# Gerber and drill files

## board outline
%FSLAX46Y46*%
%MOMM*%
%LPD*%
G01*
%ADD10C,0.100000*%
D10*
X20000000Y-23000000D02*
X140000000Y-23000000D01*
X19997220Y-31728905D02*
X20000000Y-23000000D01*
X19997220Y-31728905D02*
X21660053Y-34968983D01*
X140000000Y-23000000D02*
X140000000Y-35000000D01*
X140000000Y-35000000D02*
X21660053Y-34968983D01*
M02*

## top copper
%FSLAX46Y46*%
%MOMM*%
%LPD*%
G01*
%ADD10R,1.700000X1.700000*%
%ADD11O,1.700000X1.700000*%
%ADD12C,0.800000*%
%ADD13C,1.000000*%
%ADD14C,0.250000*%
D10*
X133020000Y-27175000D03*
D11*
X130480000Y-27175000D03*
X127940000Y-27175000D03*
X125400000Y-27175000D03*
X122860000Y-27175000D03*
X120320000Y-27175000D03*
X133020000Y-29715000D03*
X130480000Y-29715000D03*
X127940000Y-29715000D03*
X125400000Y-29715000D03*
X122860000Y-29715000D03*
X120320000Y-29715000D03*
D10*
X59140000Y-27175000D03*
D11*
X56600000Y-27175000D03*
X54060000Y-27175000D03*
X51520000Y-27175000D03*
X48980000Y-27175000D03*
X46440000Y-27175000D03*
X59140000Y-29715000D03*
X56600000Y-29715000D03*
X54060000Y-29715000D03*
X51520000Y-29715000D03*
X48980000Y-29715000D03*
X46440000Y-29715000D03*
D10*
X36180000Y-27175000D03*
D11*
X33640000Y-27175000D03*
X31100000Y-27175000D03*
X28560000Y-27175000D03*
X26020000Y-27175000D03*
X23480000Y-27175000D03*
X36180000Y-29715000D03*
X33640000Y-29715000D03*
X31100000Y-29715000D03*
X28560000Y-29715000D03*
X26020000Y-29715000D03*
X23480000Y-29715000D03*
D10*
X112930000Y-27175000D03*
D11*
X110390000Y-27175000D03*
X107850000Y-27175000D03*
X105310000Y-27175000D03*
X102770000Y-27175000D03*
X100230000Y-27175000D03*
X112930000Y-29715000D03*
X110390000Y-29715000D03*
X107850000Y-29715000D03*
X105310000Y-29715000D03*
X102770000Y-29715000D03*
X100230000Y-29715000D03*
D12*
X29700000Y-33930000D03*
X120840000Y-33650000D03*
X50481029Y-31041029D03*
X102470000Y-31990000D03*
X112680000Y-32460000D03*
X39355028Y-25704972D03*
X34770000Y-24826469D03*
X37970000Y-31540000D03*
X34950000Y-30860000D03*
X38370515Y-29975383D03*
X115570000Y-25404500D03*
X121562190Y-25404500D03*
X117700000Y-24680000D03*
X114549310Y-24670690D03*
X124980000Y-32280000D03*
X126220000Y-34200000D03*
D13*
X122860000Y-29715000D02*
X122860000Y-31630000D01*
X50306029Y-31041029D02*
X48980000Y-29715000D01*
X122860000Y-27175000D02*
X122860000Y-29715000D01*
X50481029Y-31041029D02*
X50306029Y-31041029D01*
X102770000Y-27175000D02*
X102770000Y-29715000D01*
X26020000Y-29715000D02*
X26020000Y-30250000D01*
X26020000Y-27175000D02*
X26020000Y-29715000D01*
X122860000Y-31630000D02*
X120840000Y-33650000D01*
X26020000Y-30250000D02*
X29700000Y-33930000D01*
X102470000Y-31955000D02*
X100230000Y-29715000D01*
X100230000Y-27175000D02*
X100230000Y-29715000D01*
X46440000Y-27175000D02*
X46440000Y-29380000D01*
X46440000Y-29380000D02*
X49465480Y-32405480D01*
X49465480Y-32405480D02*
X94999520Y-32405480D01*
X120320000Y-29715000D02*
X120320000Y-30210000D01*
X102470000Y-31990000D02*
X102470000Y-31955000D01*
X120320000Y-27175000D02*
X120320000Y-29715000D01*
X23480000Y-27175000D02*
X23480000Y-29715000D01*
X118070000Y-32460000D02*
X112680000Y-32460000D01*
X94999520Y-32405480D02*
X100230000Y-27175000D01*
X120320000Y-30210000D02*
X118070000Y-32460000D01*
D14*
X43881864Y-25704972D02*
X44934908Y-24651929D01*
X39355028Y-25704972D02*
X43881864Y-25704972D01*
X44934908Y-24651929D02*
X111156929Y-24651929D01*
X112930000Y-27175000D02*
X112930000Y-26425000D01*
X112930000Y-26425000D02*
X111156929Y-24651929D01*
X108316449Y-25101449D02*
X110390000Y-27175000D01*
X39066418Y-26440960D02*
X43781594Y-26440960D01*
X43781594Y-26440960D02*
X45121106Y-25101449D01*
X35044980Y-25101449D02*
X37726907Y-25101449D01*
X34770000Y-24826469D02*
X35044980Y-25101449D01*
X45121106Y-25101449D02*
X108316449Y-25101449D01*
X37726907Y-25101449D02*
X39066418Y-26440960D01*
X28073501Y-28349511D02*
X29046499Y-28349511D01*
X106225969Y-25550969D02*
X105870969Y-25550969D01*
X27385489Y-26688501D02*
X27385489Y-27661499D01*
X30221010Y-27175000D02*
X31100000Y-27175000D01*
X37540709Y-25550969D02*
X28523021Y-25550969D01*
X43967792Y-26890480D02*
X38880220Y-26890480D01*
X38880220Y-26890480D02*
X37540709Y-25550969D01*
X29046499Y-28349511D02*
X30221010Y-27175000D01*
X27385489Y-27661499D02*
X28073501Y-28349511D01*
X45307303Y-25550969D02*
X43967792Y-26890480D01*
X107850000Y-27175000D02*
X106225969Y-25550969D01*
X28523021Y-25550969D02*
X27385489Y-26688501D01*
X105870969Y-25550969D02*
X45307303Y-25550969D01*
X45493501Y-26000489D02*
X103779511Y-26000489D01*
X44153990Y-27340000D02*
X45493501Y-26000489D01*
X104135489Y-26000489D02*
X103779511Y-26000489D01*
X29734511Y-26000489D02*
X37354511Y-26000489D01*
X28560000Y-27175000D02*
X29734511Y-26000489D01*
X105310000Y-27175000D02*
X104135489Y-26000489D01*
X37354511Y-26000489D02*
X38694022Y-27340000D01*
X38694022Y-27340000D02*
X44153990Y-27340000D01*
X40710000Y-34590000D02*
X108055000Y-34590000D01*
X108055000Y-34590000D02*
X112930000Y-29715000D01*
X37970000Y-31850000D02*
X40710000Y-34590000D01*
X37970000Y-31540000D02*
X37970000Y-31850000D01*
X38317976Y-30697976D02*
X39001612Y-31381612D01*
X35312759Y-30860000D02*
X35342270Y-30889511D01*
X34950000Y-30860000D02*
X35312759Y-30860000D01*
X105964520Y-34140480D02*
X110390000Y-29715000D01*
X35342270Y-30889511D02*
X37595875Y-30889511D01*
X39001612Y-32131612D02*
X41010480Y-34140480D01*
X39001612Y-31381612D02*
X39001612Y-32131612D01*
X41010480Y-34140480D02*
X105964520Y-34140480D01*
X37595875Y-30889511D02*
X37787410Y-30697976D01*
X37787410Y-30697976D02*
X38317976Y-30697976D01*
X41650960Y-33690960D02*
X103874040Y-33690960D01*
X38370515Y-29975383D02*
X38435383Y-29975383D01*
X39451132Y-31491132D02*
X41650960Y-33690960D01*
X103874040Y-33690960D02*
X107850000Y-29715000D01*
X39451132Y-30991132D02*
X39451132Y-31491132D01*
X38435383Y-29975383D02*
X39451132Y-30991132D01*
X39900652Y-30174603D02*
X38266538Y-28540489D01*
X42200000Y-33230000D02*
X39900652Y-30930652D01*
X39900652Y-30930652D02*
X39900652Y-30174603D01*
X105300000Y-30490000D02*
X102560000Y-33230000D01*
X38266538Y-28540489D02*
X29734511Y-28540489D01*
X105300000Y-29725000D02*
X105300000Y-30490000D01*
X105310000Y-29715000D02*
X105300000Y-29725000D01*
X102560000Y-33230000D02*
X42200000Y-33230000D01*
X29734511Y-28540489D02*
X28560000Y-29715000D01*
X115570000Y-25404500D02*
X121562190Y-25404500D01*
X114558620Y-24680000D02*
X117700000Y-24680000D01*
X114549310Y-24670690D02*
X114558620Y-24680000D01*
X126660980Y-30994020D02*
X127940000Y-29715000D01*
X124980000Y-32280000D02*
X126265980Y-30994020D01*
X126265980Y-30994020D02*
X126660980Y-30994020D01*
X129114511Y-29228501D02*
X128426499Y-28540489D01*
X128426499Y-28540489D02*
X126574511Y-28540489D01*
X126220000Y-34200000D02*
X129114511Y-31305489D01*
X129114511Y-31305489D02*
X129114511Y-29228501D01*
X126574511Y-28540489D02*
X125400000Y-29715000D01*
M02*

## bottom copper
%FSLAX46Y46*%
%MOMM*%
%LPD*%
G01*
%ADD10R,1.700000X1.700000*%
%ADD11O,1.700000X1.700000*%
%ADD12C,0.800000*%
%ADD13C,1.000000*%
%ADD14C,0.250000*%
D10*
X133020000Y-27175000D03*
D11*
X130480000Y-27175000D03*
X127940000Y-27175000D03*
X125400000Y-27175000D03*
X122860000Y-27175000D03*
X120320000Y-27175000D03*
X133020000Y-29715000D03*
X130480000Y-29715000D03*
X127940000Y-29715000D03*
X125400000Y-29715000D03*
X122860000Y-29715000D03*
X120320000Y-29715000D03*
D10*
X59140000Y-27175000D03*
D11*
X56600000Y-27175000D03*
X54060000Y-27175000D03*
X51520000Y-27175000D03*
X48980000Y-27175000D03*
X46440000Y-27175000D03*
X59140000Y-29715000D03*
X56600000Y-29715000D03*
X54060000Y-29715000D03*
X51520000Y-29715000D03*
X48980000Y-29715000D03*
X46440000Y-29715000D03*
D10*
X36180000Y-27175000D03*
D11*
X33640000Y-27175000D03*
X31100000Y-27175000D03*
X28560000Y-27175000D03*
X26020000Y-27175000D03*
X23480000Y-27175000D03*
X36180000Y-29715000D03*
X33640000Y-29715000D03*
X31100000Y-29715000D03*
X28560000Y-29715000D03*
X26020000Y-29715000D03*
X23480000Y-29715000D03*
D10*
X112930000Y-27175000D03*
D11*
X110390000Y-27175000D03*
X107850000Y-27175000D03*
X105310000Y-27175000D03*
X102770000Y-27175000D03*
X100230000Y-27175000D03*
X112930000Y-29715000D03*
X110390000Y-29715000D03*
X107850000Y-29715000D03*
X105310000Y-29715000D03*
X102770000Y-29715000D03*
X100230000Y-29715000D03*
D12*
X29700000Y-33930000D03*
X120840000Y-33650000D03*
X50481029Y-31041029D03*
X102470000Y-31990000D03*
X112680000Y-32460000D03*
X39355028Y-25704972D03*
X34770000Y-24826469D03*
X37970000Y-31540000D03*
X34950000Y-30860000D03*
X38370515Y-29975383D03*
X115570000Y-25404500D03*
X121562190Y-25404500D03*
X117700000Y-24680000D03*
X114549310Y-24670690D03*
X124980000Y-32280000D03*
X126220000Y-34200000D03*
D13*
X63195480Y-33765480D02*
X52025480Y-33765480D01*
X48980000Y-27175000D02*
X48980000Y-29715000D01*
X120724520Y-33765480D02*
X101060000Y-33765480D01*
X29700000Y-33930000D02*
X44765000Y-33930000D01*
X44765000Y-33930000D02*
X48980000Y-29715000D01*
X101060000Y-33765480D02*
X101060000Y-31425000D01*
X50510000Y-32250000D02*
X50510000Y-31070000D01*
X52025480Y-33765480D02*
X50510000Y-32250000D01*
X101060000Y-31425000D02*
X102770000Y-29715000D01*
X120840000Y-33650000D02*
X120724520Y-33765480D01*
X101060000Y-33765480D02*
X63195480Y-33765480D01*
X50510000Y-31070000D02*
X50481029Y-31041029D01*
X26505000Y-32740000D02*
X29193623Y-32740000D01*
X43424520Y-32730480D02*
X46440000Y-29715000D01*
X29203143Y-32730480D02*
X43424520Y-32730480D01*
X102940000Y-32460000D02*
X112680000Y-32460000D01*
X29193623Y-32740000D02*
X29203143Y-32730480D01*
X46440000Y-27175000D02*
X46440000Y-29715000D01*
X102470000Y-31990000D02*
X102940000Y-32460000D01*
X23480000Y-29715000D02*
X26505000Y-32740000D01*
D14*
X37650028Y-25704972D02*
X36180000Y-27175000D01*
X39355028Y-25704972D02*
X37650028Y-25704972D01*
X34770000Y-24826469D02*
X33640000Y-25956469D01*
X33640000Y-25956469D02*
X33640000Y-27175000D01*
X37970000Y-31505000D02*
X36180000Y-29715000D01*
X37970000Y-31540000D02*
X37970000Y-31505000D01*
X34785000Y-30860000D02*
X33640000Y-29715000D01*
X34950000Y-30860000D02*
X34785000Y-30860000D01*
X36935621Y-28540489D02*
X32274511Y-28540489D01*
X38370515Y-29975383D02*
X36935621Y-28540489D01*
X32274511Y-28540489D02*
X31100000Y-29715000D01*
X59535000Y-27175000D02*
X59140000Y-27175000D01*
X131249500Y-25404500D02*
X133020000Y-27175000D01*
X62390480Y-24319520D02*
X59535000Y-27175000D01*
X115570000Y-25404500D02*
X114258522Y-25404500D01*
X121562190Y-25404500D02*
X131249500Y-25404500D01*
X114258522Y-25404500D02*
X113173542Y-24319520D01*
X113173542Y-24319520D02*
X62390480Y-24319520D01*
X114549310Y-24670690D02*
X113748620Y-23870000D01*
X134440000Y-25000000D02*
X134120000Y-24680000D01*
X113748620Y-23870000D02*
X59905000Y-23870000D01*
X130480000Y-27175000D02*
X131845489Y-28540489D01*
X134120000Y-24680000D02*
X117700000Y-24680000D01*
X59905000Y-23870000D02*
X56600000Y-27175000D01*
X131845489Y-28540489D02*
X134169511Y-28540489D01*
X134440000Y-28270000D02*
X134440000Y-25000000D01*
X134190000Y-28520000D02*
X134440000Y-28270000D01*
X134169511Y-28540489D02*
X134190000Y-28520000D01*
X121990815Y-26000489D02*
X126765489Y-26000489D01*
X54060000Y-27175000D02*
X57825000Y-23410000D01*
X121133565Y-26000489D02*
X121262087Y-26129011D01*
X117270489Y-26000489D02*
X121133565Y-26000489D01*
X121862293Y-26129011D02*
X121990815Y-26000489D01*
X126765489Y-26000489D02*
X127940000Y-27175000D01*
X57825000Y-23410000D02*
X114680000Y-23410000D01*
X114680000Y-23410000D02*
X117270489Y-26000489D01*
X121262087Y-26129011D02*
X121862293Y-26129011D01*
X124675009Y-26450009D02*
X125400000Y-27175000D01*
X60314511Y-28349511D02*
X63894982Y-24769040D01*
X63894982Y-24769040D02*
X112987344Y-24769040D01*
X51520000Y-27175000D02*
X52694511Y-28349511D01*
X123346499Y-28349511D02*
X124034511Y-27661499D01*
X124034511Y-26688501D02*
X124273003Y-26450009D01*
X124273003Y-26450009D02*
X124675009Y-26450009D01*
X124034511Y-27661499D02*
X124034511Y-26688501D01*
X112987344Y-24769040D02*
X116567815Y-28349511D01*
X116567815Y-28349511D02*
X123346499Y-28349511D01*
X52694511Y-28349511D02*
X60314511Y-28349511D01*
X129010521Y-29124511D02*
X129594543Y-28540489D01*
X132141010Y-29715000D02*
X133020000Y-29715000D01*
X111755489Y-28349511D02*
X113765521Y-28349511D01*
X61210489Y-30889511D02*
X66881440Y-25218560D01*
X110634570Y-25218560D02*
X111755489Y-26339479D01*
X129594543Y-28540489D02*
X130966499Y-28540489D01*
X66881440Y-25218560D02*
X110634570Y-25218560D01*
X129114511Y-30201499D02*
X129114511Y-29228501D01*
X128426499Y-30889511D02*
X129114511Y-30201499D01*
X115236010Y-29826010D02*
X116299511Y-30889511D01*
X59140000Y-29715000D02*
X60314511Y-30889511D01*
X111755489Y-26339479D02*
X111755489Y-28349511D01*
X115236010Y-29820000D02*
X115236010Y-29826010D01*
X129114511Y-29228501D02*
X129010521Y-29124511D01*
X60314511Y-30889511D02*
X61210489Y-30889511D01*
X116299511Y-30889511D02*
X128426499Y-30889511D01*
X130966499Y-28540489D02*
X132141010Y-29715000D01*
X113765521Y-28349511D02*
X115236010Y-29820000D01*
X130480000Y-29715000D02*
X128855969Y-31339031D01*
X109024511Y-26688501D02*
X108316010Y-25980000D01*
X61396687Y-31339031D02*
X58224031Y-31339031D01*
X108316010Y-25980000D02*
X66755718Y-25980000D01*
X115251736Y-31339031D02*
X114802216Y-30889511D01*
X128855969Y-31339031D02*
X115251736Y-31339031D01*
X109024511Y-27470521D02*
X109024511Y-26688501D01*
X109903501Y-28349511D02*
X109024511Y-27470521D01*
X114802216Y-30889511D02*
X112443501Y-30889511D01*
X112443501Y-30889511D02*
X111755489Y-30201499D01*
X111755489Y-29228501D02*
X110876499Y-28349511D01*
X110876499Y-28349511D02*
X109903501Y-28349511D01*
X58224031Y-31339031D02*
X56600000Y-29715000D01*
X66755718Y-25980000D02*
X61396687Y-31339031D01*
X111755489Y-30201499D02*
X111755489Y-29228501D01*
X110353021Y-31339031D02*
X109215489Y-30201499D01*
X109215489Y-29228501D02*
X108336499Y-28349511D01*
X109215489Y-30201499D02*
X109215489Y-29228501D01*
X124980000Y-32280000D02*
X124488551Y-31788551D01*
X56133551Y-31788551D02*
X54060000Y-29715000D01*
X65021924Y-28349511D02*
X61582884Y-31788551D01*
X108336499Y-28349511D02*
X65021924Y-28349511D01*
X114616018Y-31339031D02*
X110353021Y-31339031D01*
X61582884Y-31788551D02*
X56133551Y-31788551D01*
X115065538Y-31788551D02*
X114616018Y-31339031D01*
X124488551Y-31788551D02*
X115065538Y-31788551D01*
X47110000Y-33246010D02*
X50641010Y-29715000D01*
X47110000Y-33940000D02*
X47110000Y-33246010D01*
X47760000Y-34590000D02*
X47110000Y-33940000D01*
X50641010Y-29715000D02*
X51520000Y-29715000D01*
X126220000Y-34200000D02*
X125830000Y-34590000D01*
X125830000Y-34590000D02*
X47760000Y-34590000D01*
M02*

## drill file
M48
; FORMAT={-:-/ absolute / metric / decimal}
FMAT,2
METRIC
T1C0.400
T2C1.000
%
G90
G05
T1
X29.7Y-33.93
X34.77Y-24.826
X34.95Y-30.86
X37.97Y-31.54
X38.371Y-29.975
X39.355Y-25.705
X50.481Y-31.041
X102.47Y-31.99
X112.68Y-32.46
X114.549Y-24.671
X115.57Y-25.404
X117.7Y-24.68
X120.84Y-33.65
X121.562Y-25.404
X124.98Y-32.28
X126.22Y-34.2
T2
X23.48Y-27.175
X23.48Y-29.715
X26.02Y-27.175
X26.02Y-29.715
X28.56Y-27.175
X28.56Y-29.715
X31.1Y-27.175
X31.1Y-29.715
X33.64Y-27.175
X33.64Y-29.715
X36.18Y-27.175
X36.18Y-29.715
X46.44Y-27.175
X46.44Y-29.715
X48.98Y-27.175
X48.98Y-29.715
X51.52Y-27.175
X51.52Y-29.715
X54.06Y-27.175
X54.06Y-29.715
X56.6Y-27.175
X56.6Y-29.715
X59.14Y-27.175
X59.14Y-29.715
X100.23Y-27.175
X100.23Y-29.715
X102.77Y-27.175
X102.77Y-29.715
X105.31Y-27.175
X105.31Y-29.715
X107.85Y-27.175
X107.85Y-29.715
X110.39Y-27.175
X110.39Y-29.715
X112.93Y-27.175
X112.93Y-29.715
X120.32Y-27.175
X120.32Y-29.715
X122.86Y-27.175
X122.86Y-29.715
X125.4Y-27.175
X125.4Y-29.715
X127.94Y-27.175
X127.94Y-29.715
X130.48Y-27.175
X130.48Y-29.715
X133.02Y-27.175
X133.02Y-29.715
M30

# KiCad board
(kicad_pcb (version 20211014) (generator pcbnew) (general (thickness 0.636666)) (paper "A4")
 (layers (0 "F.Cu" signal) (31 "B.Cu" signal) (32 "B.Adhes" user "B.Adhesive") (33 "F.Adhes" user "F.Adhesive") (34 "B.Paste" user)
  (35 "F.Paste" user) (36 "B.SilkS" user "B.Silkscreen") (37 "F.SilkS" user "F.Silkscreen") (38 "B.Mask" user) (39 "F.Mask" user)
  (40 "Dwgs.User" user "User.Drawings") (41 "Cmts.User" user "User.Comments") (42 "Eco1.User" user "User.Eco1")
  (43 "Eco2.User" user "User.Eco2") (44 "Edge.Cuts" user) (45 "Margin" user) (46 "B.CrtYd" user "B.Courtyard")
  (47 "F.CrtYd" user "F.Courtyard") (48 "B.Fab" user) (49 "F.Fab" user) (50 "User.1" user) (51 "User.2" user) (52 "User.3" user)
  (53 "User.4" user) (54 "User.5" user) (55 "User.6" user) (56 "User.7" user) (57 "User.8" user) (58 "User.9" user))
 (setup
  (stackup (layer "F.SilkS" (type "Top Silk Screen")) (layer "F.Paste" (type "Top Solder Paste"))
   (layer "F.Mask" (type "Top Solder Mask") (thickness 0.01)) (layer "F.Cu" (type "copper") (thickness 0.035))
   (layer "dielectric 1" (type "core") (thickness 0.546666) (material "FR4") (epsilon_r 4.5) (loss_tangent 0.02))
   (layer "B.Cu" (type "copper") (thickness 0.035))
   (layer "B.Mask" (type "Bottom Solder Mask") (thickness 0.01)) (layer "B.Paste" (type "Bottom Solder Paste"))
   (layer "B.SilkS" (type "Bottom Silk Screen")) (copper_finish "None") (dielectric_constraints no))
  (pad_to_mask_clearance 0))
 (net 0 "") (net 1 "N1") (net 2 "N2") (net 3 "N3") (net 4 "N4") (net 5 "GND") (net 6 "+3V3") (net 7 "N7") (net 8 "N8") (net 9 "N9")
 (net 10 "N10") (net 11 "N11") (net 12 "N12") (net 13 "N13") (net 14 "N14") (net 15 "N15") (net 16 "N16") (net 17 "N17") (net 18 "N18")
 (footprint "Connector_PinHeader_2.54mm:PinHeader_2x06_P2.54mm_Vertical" (layer "F.Cu") (at 133.02 27.175 -90)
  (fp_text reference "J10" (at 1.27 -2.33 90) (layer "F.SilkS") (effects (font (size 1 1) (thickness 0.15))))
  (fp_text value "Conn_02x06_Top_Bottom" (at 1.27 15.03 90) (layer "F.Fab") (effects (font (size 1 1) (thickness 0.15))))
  (pad "1" thru_hole rect (at 0 0 270) (size 1.7 1.7) (drill 1) (layers *.Cu *.Mask) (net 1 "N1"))
  (pad "2" thru_hole oval (at 0 2.54 270) (size 1.7 1.7) (drill 1) (layers *.Cu *.Mask) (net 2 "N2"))
  (pad "3" thru_hole oval (at 0 5.08 270) (size 1.7 1.7) (drill 1) (layers *.Cu *.Mask) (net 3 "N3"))
  (pad "4" thru_hole oval (at 0 7.62 270) (size 1.7 1.7) (drill 1) (layers *.Cu *.Mask) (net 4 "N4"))
  (pad "5" thru_hole oval (at 0 10.16 270) (size 1.7 1.7) (drill 1) (layers *.Cu *.Mask) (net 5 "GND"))
  (pad "6" thru_hole oval (at 0 12.7 270) (size 1.7 1.7) (drill 1) (layers *.Cu *.Mask) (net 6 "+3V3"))
  (pad "7" thru_hole oval (at 2.54 0 270) (size 1.7 1.7) (drill 1) (layers *.Cu *.Mask) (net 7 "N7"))
  (pad "8" thru_hole oval (at 2.54 2.54 270) (size 1.7 1.7) (drill 1) (layers *.Cu *.Mask) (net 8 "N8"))
  (pad "9" thru_hole oval (at 2.54 5.08 270) (size 1.7 1.7) (drill 1) (layers *.Cu *.Mask) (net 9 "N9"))
  (pad "10" thru_hole oval (at 2.54 7.62 270) (size 1.7 1.7) (drill 1) (layers *.Cu *.Mask) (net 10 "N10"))
  (pad "11" thru_hole oval (at 2.54 10.16 270) (size 1.7 1.7) (drill 1) (layers *.Cu *.Mask) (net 5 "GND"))
  (pad "12" thru_hole oval (at 2.54 12.7 270) (size 1.7 1.7) (drill 1) (layers *.Cu *.Mask) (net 6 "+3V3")))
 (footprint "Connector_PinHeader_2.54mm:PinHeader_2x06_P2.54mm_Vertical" (layer "F.Cu") (at 59.14 27.175 -90)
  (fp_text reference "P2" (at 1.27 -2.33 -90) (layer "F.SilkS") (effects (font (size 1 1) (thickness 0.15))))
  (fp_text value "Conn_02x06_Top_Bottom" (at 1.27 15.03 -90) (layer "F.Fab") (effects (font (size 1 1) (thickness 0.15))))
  (pad "1" thru_hole rect (at 0 0 270) (size 1.7 1.7) (drill 1) (layers *.Cu *.Mask) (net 1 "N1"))
  (pad "2" thru_hole oval (at 0 2.54 270) (size 1.7 1.7) (drill 1) (layers *.Cu *.Mask) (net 2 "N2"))
  (pad "3" thru_hole oval (at 0 5.08 270) (size 1.7 1.7) (drill 1) (layers *.Cu *.Mask) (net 3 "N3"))
  (pad "4" thru_hole oval (at 0 7.62 270) (size 1.7 1.7) (drill 1) (layers *.Cu *.Mask) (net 4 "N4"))
  (pad "5" thru_hole oval (at 0 10.16 270) (size 1.7 1.7) (drill 1) (layers *.Cu *.Mask) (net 5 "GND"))
  (pad "6" thru_hole oval (at 0 12.7 270) (size 1.7 1.7) (drill 1) (layers *.Cu *.Mask) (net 6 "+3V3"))
  (pad "7" thru_hole oval (at 2.54 0 270) (size 1.7 1.7) (drill 1) (layers *.Cu *.Mask) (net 7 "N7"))
  (pad "8" thru_hole oval (at 2.54 2.54 270) (size 1.7 1.7) (drill 1) (layers *.Cu *.Mask) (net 8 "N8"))
  (pad "9" thru_hole oval (at 2.54 5.08 270) (size 1.7 1.7) (drill 1) (layers *.Cu *.Mask) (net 9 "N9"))
  (pad "10" thru_hole oval (at 2.54 7.62 270) (size 1.7 1.7) (drill 1) (layers *.Cu *.Mask) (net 10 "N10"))
  (pad "11" thru_hole oval (at 2.54 10.16 270) (size 1.7 1.7) (drill 1) (layers *.Cu *.Mask) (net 5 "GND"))
  (pad "12" thru_hole oval (at 2.54 12.7 270) (size 1.7 1.7) (drill 1) (layers *.Cu *.Mask) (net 6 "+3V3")))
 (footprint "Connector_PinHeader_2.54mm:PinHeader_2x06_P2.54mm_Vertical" (layer "F.Cu") (at 36.18 27.175 -90)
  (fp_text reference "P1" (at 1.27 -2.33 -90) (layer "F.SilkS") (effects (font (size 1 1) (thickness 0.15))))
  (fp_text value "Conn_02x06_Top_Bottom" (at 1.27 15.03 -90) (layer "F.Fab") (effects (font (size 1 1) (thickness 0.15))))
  (pad "1" thru_hole rect (at 0 0 270) (size 1.7 1.7) (drill 1) (layers *.Cu *.Mask) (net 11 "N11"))
  (pad "2" thru_hole oval (at 0 2.54 270) (size 1.7 1.7) (drill 1) (layers *.Cu *.Mask) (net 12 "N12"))
  (pad "3" thru_hole oval (at 0 5.08 270) (size 1.7 1.7) (drill 1) (layers *.Cu *.Mask) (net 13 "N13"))
  (pad "4" thru_hole oval (at 0 7.62 270) (size 1.7 1.7) (drill 1) (layers *.Cu *.Mask) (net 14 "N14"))
  (pad "5" thru_hole oval (at 0 10.16 270) (size 1.7 1.7) (drill 1) (layers *.Cu *.Mask) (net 5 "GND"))
  (pad "6" thru_hole oval (at 0 12.7 270) (size 1.7 1.7) (drill 1) (layers *.Cu *.Mask) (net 6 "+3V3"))
  (pad "7" thru_hole oval (at 2.54 0 270) (size 1.7 1.7) (drill 1) (layers *.Cu *.Mask) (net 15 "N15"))
  (pad "8" thru_hole oval (at 2.54 2.54 270) (size 1.7 1.7) (drill 1) (layers *.Cu *.Mask) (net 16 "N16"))
  (pad "9" thru_hole oval (at 2.54 5.08 270) (size 1.7 1.7) (drill 1) (layers *.Cu *.Mask) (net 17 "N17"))
  (pad "10" thru_hole oval (at 2.54 7.62 270) (size 1.7 1.7) (drill 1) (layers *.Cu *.Mask) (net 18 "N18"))
  (pad "11" thru_hole oval (at 2.54 10.16 270) (size 1.7 1.7) (drill 1) (layers *.Cu *.Mask) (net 5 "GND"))
  (pad "12" thru_hole oval (at 2.54 12.7 270) (size 1.7 1.7) (drill 1) (layers *.Cu *.Mask) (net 6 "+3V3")))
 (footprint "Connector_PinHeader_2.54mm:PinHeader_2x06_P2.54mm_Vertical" (layer "F.Cu") (at 112.93 27.175 -90)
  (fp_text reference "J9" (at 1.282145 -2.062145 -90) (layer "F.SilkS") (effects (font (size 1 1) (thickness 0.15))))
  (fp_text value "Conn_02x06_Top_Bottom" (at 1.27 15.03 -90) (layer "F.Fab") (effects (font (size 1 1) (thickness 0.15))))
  (pad "1" thru_hole rect (at 0 0 270) (size 1.7 1.7) (drill 1) (layers *.Cu *.Mask) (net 11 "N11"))
  (pad "2" thru_hole oval (at 0 2.54 270) (size 1.7 1.7) (drill 1) (layers *.Cu *.Mask) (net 12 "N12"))
  (pad "3" thru_hole oval (at 0 5.08 270) (size 1.7 1.7) (drill 1) (layers *.Cu *.Mask) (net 13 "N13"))
  (pad "4" thru_hole oval (at 0 7.62 270) (size 1.7 1.7) (drill 1) (layers *.Cu *.Mask) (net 14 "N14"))
  (pad "5" thru_hole oval (at 0 10.16 270) (size 1.7 1.7) (drill 1) (layers *.Cu *.Mask) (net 5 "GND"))
  (pad "6" thru_hole oval (at 0 12.7 270) (size 1.7 1.7) (drill 1) (layers *.Cu *.Mask) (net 6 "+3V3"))
  (pad "7" thru_hole oval (at 2.54 0 270) (size 1.7 1.7) (drill 1) (layers *.Cu *.Mask) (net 15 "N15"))
  (pad "8" thru_hole oval (at 2.54 2.54 270) (size 1.7 1.7) (drill 1) (layers *.Cu *.Mask) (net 16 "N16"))
  (pad "9" thru_hole oval (at 2.54 5.08 270) (size 1.7 1.7) (drill 1) (layers *.Cu *.Mask) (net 17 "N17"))
  (pad "10" thru_hole oval (at 2.54 7.62 270) (size 1.7 1.7) (drill 1) (layers *.Cu *.Mask) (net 18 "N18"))
  (pad "11" thru_hole oval (at 2.54 10.16 270) (size 1.7 1.7) (drill 1) (layers *.Cu *.Mask) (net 5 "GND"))
  (pad "12" thru_hole oval (at 2.54 12.7 270) (size 1.7 1.7) (drill 1) (layers *.Cu *.Mask) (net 6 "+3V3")))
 (gr_line (start 20 23) (end 140 23) (layer "Edge.Cuts") (width 0.1))
 (gr_line (start 19.99722 31.728905) (end 20 23) (layer "Edge.Cuts") (width 0.1))
 (gr_line (start 19.99722 31.728905) (end 21.660053 34.968983) (layer "Edge.Cuts") (width 0.1))
 (gr_line (start 140 23) (end 140 35) (layer "Edge.Cuts") (width 0.1))
 (gr_line (start 140 35) (end 21.660053 34.968983) (layer "Edge.Cuts") (width 0.1))
 (segment (start 122.86 29.715) (end 122.86 31.63) (width 1) (layer "F.Cu") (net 5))
 (segment (start 50.306029 31.041029) (end 48.98 29.715) (width 1) (layer "F.Cu") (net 5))
 (segment (start 122.86 27.175) (end 122.86 29.715) (width 1) (layer "F.Cu") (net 5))
 (segment (start 50.481029 31.041029) (end 50.306029 31.041029) (width 1) (layer "F.Cu") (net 5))
 (segment (start 102.77 27.175) (end 102.77 29.715) (width 1) (layer "F.Cu") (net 5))
 (segment (start 26.02 29.715) (end 26.02 30.25) (width 1) (layer "F.Cu") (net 5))
 (segment (start 26.02 27.175) (end 26.02 29.715) (width 1) (layer "F.Cu") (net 5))
 (segment (start 122.86 31.63) (end 120.84 33.65) (width 1) (layer "F.Cu") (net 5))
 (segment (start 26.02 30.25) (end 29.7 33.93) (width 1) (layer "F.Cu") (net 5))
 (via (at 29.7 33.93) (size 0.8) (drill 0.4) (layers "F.Cu" "B.Cu") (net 5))
 (via (at 120.84 33.65) (size 0.8) (drill 0.4) (layers "F.Cu" "B.Cu") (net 5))
 (via (at 50.481029 31.041029) (size 0.8) (drill 0.4) (layers "F.Cu" "B.Cu") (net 5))
 (segment (start 63.19548 33.76548) (end 52.02548 33.76548) (width 1) (layer "B.Cu") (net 5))
 (segment (start 48.98 27.175) (end 48.98 29.715) (width 1) (layer "B.Cu") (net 5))
 (segment (start 120.72452 33.76548) (end 101.06 33.76548) (width 1) (layer "B.Cu") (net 5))
 (segment (start 29.7 33.93) (end 44.765 33.93) (width 1) (layer "B.Cu") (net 5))
 (segment (start 44.765 33.93) (end 48.98 29.715) (width 1) (layer "B.Cu") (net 5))
 (segment (start 101.06 33.76548) (end 101.06 31.425) (width 1) (layer "B.Cu") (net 5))
 (segment (start 50.51 32.25) (end 50.51 31.07) (width 1) (layer "B.Cu") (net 5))
 (segment (start 52.02548 33.76548) (end 50.51 32.25) (width 1) (layer "B.Cu") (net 5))
 (segment (start 101.06 31.425) (end 102.77 29.715) (width 1) (layer "B.Cu") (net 5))
 (segment (start 120.84 33.65) (end 120.72452 33.76548) (width 1) (layer "B.Cu") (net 5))
 (segment (start 101.06 33.76548) (end 63.19548 33.76548) (width 1) (layer "B.Cu") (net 5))
 (segment (start 50.51 31.07) (end 50.481029 31.041029) (width 1) (layer "B.Cu") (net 5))
 (segment (start 102.47 31.955) (end 100.23 29.715) (width 1) (layer "F.Cu") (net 6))
 (segment (start 100.23 27.175) (end 100.23 29.715) (width 1) (layer "F.Cu") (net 6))
 (segment (start 46.44 27.175) (end 46.44 29.38) (width 1) (layer "F.Cu") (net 6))
 (segment (start 46.44 29.38) (end 49.46548 32.40548) (width 1) (layer "F.Cu") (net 6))
 (segment (start 49.46548 32.40548) (end 94.99952 32.40548) (width 1) (layer "F.Cu") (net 6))
 (segment (start 120.32 29.715) (end 120.32 30.21) (width 1) (layer "F.Cu") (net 6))
 (segment (start 102.47 31.99) (end 102.47 31.955) (width 1) (layer "F.Cu") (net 6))
 (segment (start 120.32 27.175) (end 120.32 29.715) (width 1) (layer "F.Cu") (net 6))
 (segment (start 23.48 27.175) (end 23.48 29.715) (width 1) (layer "F.Cu") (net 6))
 (segment (start 118.07 32.46) (end 112.68 32.46) (width 1) (layer "F.Cu") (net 6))
 (segment (start 94.99952 32.40548) (end 100.23 27.175) (width 1) (layer "F.Cu") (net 6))
 (segment (start 120.32 30.21) (end 118.07 32.46) (width 1) (layer "F.Cu") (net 6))
 (via (at 102.47 31.99) (size 0.8) (drill 0.4) (layers "F.Cu" "B.Cu") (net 6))
 (via (at 112.68 32.46) (size 0.8) (drill 0.4) (layers "F.Cu" "B.Cu") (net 6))
 (segment (start 26.505 32.74) (end 29.193623 32.74) (width 1) (layer "B.Cu") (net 6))
 (segment (start 43.42452 32.73048) (end 46.44 29.715) (width 1) (layer "B.Cu") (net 6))
 (segment (start 29.203143 32.73048) (end 43.42452 32.73048) (width 1) (layer "B.Cu") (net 6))
 (segment (start 102.94 32.46) (end 112.68 32.46) (width 1) (layer "B.Cu") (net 6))
 (segment (start 29.193623 32.74) (end 29.203143 32.73048) (width 1) (layer "B.Cu") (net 6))
 (segment (start 46.44 27.175) (end 46.44 29.715) (width 1) (layer "B.Cu") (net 6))
 (segment (start 102.47 31.99) (end 102.94 32.46) (width 1) (layer "B.Cu") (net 6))
 (segment (start 23.48 29.715) (end 26.505 32.74) (width 1) (layer "B.Cu") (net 6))
 (segment (start 43.881864 25.704972) (end 44.934908 24.651929) (width 0.25) (layer "F.Cu") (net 11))
 (segment (start 39.355028 25.704972) (end 43.881864 25.704972) (width 0.25) (layer "F.Cu") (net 11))
 (segment (start 44.934908 24.651929) (end 111.156929 24.651929) (width 0.25) (layer "F.Cu") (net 11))
 (segment (start 112.93 27.175) (end 112.93 26.425) (width 0.25) (layer "F.Cu") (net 11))
 (segment (start 112.93 26.425) (end 111.156929 24.651929) (width 0.25) (layer "F.Cu") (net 11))
 (via (at 39.355028 25.704972) (size 0.8) (drill 0.4) (layers "F.Cu" "B.Cu") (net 11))
 (segment (start 37.650028 25.704972) (end 36.18 27.175) (width 0.25) (layer "B.Cu") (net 11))
 (segment (start 39.355028 25.704972) (end 37.650028 25.704972) (width 0.25) (layer "B.Cu") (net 11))
 (segment (start 108.316449 25.101449) (end 110.39 27.175) (width 0.25) (layer "F.Cu") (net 12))
 (segment (start 39.066418 26.44096) (end 43.781594 26.44096) (width 0.25) (layer "F.Cu") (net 12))
 (segment (start 43.781594 26.44096) (end 45.121106 25.101449) (width 0.25) (layer "F.Cu") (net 12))
 (segment (start 35.04498 25.101449) (end 37.726907 25.101449) (width 0.25) (layer "F.Cu") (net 12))
 (segment (start 34.77 24.826469) (end 35.04498 25.101449) (width 0.25) (layer "F.Cu") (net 12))
 (segment (start 45.121106 25.101449) (end 108.316449 25.101449) (width 0.25) (layer "F.Cu") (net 12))
 (segment (start 37.726907 25.101449) (end 39.066418 26.44096) (width 0.25) (layer "F.Cu") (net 12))
 (via (at 34.77 24.826469) (size 0.8) (drill 0.4) (layers "F.Cu" "B.Cu") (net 12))
 (segment (start 34.77 24.826469) (end 33.64 25.956469) (width 0.25) (layer "B.Cu") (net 12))
 (segment (start 33.64 25.956469) (end 33.64 27.175) (width 0.25) (layer "B.Cu") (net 12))
 (segment (start 28.073501 28.349511) (end 29.046499 28.349511) (width 0.25) (layer "F.Cu") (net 13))
 (segment (start 106.225969 25.550969) (end 105.870969 25.550969) (width 0.25) (layer "F.Cu") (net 13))
 (segment (start 27.385489 26.688501) (end 27.385489 27.661499) (width 0.25) (layer "F.Cu") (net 13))
 (segment (start 30.22101 27.175) (end 31.1 27.175) (width 0.25) (layer "F.Cu") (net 13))
 (segment (start 37.540709 25.550969) (end 28.523021 25.550969) (width 0.25) (layer "F.Cu") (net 13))
 (segment (start 43.967792 26.89048) (end 38.88022 26.89048) (width 0.25) (layer "F.Cu") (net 13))
 (segment (start 38.88022 26.89048) (end 37.540709 25.550969) (width 0.25) (layer "F.Cu") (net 13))
 (segment (start 29.046499 28.349511) (end 30.22101 27.175) (width 0.25) (layer "F.Cu") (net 13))
 (segment (start 27.385489 27.661499) (end 28.073501 28.349511) (width 0.25) (layer "F.Cu") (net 13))
 (segment (start 45.307303 25.550969) (end 43.967792 26.89048) (width 0.25) (layer "F.Cu") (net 13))
 (segment (start 107.85 27.175) (end 106.225969 25.550969) (width 0.25) (layer "F.Cu") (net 13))
 (segment (start 28.523021 25.550969) (end 27.385489 26.688501) (width 0.25) (layer "F.Cu") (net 13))
 (segment (start 105.870969 25.550969) (end 45.307303 25.550969) (width 0.25) (layer "F.Cu") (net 13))
 (segment (start 45.493501 26.000489) (end 103.779511 26.000489) (width 0.25) (layer "F.Cu") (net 14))
 (segment (start 44.15399 27.34) (end 45.493501 26.000489) (width 0.25) (layer "F.Cu") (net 14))
 (segment (start 104.135489 26.000489) (end 103.779511 26.000489) (width 0.25) (layer "F.Cu") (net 14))
 (segment (start 29.734511 26.000489) (end 37.354511 26.000489) (width 0.25) (layer "F.Cu") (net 14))
 (segment (start 28.56 27.175) (end 29.734511 26.000489) (width 0.25) (layer "F.Cu") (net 14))
 (segment (start 105.31 27.175) (end 104.135489 26.000489) (width 0.25) (layer "F.Cu") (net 14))
 (segment (start 37.354511 26.000489) (end 38.694022 27.34) (width 0.25) (layer "F.Cu") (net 14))
 (segment (start 38.694022 27.34) (end 44.15399 27.34) (width 0.25) (layer "F.Cu") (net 14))
 (segment (start 40.71 34.59) (end 108.055 34.59) (width 0.25) (layer "F.Cu") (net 15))
 (segment (start 108.055 34.59) (end 112.93 29.715) (width 0.25) (layer "F.Cu") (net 15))
 (segment (start 37.97 31.85) (end 40.71 34.59) (width 0.25) (layer "F.Cu") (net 15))
 (segment (start 37.97 31.54) (end 37.97 31.85) (width 0.25) (layer "F.Cu") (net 15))
 (via (at 37.97 31.54) (size 0.8) (drill 0.4) (layers "F.Cu" "B.Cu") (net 15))
 (segment (start 37.97 31.505) (end 36.18 29.715) (width 0.25) (layer "B.Cu") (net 15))
 (segment (start 37.97 31.54) (end 37.97 31.505) (width 0.25) (layer "B.Cu") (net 15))
 (segment (start 38.317976 30.697976) (end 39.001612 31.381612) (width 0.25) (layer "F.Cu") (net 16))
 (segment (start 35.312759 30.86) (end 35.34227 30.889511) (width 0.25) (layer "F.Cu") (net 16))
 (segment (start 34.95 30.86) (end 35.312759 30.86) (width 0.25) (layer "F.Cu") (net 16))
 (segment (start 105.96452 34.14048) (end 110.39 29.715) (width 0.25) (layer "F.Cu") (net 16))
 (segment (start 35.34227 30.889511) (end 37.595875 30.889511) (width 0.25) (layer "F.Cu") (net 16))
 (segment (start 39.001612 32.131612) (end 41.01048 34.14048) (width 0.25) (layer "F.Cu") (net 16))
 (segment (start 39.001612 31.381612) (end 39.001612 32.131612) (width 0.25) (layer "F.Cu") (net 16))
 (segment (start 41.01048 34.14048) (end 105.96452 34.14048) (width 0.25) (layer "F.Cu") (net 16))
 (segment (start 37.595875 30.889511) (end 37.78741 30.697976) (width 0.25) (layer "F.Cu") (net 16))
 (segment (start 37.78741 30.697976) (end 38.317976 30.697976) (width 0.25) (layer "F.Cu") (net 16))
 (via (at 34.95 30.86) (size 0.8) (drill 0.4) (layers "F.Cu" "B.Cu") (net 16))
 (segment (start 34.785 30.86) (end 33.64 29.715) (width 0.25) (layer "B.Cu") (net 16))
 (segment (start 34.95 30.86) (end 34.785 30.86) (width 0.25) (layer "B.Cu") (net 16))
 (segment (start 41.65096 33.69096) (end 103.87404 33.69096) (width 0.25) (layer "F.Cu") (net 17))
 (segment (start 38.370515 29.975383) (end 38.435383 29.975383) (width 0.25) (layer "F.Cu") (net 17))
 (segment (start 39.451132 31.491132) (end 41.65096 33.69096) (width 0.25) (layer "F.Cu") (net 17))
 (segment (start 103.87404 33.69096) (end 107.85 29.715) (width 0.25) (layer "F.Cu") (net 17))
 (segment (start 39.451132 30.991132) (end 39.451132 31.491132) (width 0.25) (layer "F.Cu") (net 17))
 (segment (start 38.435383 29.975383) (end 39.451132 30.991132) (width 0.25) (layer "F.Cu") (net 17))
 (via (at 38.370515 29.975383) (size 0.8) (drill 0.4) (layers "F.Cu" "B.Cu") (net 17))
 (segment (start 36.935621 28.540489) (end 32.274511 28.540489) (width 0.25) (layer "B.Cu") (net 17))
 (segment (start 38.370515 29.975383) (end 36.935621 28.540489) (width 0.25) (layer "B.Cu") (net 17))
 (segment (start 32.274511 28.540489) (end 31.1 29.715) (width 0.25) (layer "B.Cu") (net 17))
 (segment (start 39.900652 30.174603) (end 38.266538 28.540489) (width 0.25) (layer "F.Cu") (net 18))
 (segment (start 42.2 33.23) (end 39.900652 30.930652) (width 0.25) (layer "F.Cu") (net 18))
 (segment (start 39.900652 30.930652) (end 39.900652 30.174603) (width 0.25) (layer "F.Cu") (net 18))
 (segment (start 105.3 30.49) (end 102.56 33.23) (width 0.25) (layer "F.Cu") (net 18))
 (segment (start 38.266538 28.540489) (end 29.734511 28.540489) (width 0.25) (layer "F.Cu") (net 18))
 (segment (start 105.3 29.725) (end 105.3 30.49) (width 0.25) (layer "F.Cu") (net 18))
 (segment (start 105.31 29.715) (end 105.3 29.725) (width 0.25) (layer "F.Cu") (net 18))
 (segment (start 102.56 33.23) (end 42.2 33.23) (width 0.25) (layer "F.Cu") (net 18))
 (segment (start 29.734511 28.540489) (end 28.56 29.715) (width 0.25) (layer "F.Cu") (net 18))
 (segment (start 115.57 25.4045) (end 121.56219 25.4045) (width 0.25) (layer "F.Cu") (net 1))
 (via (at 115.57 25.4045) (size 0.8) (drill 0.4) (layers "F.Cu" "B.Cu") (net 1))
 (via (at 121.56219 25.4045) (size 0.8) (drill 0.4) (layers "F.Cu" "B.Cu") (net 1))
 (segment (start 59.535 27.175) (end 59.14 27.175) (width 0.25) (layer "B.Cu") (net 1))
 (segment (start 131.2495 25.4045) (end 133.02 27.175) (width 0.25) (layer "B.Cu") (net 1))
 (segment (start 62.39048 24.31952) (end 59.535 27.175) (width 0.25) (layer "B.Cu") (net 1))
 (segment (start 115.57 25.4045) (end 114.258522 25.4045) (width 0.25) (layer "B.Cu") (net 1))
 (segment (start 121.56219 25.4045) (end 131.2495 25.4045) (width 0.25) (layer "B.Cu") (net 1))
 (segment (start 114.258522 25.4045) (end 113.173542 24.31952) (width 0.25) (layer "B.Cu") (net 1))
 (segment (start 113.173542 24.31952) (end 62.39048 24.31952) (width 0.25) (layer "B.Cu") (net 1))
 (segment (start 114.55862 24.68) (end 117.7 24.68) (width 0.25) (layer "F.Cu") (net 2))
 (segment (start 114.54931 24.67069) (end 114.55862 24.68) (width 0.25) (layer "F.Cu") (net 2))
 (via (at 117.7 24.68) (size 0.8) (drill 0.4) (layers "F.Cu" "B.Cu") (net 2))
 (via (at 114.54931 24.67069) (size 0.8) (drill 0.4) (layers "F.Cu" "B.Cu") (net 2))
 (segment (start 114.54931 24.67069) (end 113.74862 23.87) (width 0.25) (layer "B.Cu") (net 2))
 (segment (start 134.44 25) (end 134.12 24.68) (width 0.25) (layer "B.Cu") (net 2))
 (segment (start 113.74862 23.87) (end 59.905 23.87) (width 0.25) (layer "B.Cu") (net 2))
 (segment (start 130.48 27.175) (end 131.845489 28.540489) (width 0.25) (layer "B.Cu") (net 2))
 (segment (start 134.12 24.68) (end 117.7 24.68) (width 0.25) (layer "B.Cu") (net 2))
 (segment (start 59.905 23.87) (end 56.6 27.175) (width 0.25) (layer "B.Cu") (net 2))
 (segment (start 131.845489 28.540489) (end 134.169511 28.540489) (width 0.25) (layer "B.Cu") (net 2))
 (segment (start 134.44 28.27) (end 134.44 25) (width 0.25) (layer "B.Cu") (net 2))
 (segment (start 134.19 28.52) (end 134.44 28.27) (width 0.25) (layer "B.Cu") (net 2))
 (segment (start 134.169511 28.540489) (end 134.19 28.52) (width 0.25) (layer "B.Cu") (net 2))
 (segment (start 121.990815 26.000489) (end 126.765489 26.000489) (width 0.25) (layer "B.Cu") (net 3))
 (segment (start 54.06 27.175) (end 57.825 23.41) (width 0.25) (layer "B.Cu") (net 3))
 (segment (start 121.133565 26.000489) (end 121.262087 26.129011) (width 0.25) (layer "B.Cu") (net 3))
 (segment (start 117.270489 26.000489) (end 121.133565 26.000489) (width 0.25) (layer "B.Cu") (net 3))
 (segment (start 121.862293 26.129011) (end 121.990815 26.000489) (width 0.25) (layer "B.Cu") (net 3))
 (segment (start 126.765489 26.000489) (end 127.94 27.175) (width 0.25) (layer "B.Cu") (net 3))
 (segment (start 57.825 23.41) (end 114.68 23.41) (width 0.25) (layer "B.Cu") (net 3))
 (segment (start 114.68 23.41) (end 117.270489 26.000489) (width 0.25) (layer "B.Cu") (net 3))
 (segment (start 121.262087 26.129011) (end 121.862293 26.129011) (width 0.25) (layer "B.Cu") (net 3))
 (segment (start 124.675009 26.450009) (end 125.4 27.175) (width 0.25) (layer "B.Cu") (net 4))
 (segment (start 60.314511 28.349511) (end 63.894982 24.76904) (width 0.25) (layer "B.Cu") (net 4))
 (segment (start 63.894982 24.76904) (end 112.987344 24.76904) (width 0.25) (layer "B.Cu") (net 4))
 (segment (start 51.52 27.175) (end 52.694511 28.349511) (width 0.25) (layer "B.Cu") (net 4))
 (segment (start 123.346499 28.349511) (end 124.034511 27.661499) (width 0.25) (layer "B.Cu") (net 4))
 (segment (start 124.034511 26.688501) (end 124.273003 26.450009) (width 0.25) (layer "B.Cu") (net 4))
 (segment (start 124.273003 26.450009) (end 124.675009 26.450009) (width 0.25) (layer "B.Cu") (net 4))
 (segment (start 124.034511 27.661499) (end 124.034511 26.688501) (width 0.25) (layer "B.Cu") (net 4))
 (segment (start 112.987344 24.76904) (end 116.567815 28.349511) (width 0.25) (layer "B.Cu") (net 4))
 (segment (start 116.567815 28.349511) (end 123.346499 28.349511) (width 0.25) (layer "B.Cu") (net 4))
 (segment (start 52.694511 28.349511) (end 60.314511 28.349511) (width 0.25) (layer "B.Cu") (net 4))
 (segment (start 129.010521 29.124511) (end 129.594543 28.540489) (width 0.25) (layer "B.Cu") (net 7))
 (segment (start 132.14101 29.715) (end 133.02 29.715) (width 0.25) (layer "B.Cu") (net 7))
 (segment (start 111.755489 28.349511) (end 113.765521 28.349511) (width 0.25) (layer "B.Cu") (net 7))
 (segment (start 61.210489 30.889511) (end 66.88144 25.21856) (width 0.25) (layer "B.Cu") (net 7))
 (segment (start 110.63457 25.21856) (end 111.755489 26.339479) (width 0.25) (layer "B.Cu") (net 7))
 (segment (start 129.594543 28.540489) (end 130.966499 28.540489) (width 0.25) (layer "B.Cu") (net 7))
 (segment (start 66.88144 25.21856) (end 110.63457 25.21856) (width 0.25) (layer "B.Cu") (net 7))
 (segment (start 129.114511 30.201499) (end 129.114511 29.228501) (width 0.25) (layer "B.Cu") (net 7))
 (segment (start 128.426499 30.889511) (end 129.114511 30.201499) (width 0.25) (layer "B.Cu") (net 7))
 (segment (start 115.23601 29.82601) (end 116.299511 30.889511) (width 0.25) (layer "B.Cu") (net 7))
 (segment (start 59.14 29.715) (end 60.314511 30.889511) (width 0.25) (layer "B.Cu") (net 7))
 (segment (start 111.755489 26.339479) (end 111.755489 28.349511) (width 0.25) (layer "B.Cu") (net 7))
 (segment (start 115.23601 29.82) (end 115.23601 29.82601) (width 0.25) (layer "B.Cu") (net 7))
 (segment (start 129.114511 29.228501) (end 129.010521 29.124511) (width 0.25) (layer "B.Cu") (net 7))
 (segment (start 60.314511 30.889511) (end 61.210489 30.889511) (width 0.25) (layer "B.Cu") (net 7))
 (segment (start 116.299511 30.889511) (end 128.426499 30.889511) (width 0.25) (layer "B.Cu") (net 7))
 (segment (start 130.966499 28.540489) (end 132.14101 29.715) (width 0.25) (layer "B.Cu") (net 7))
 (segment (start 113.765521 28.349511) (end 115.23601 29.82) (width 0.25) (layer "B.Cu") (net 7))
 (segment (start 130.48 29.715) (end 128.855969 31.339031) (width 0.25) (layer "B.Cu") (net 8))
 (segment (start 109.024511 26.688501) (end 108.31601 25.98) (width 0.25) (layer "B.Cu") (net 8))
 (segment (start 61.396687 31.339031) (end 58.224031 31.339031) (width 0.25) (layer "B.Cu") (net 8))
 (segment (start 108.31601 25.98) (end 66.755718 25.98) (width 0.25) (layer "B.Cu") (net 8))
 (segment (start 115.251736 31.339031) (end 114.802216 30.889511) (width 0.25) (layer "B.Cu") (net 8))
 (segment (start 128.855969 31.339031) (end 115.251736 31.339031) (width 0.25) (layer "B.Cu") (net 8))
 (segment (start 109.024511 27.470521) (end 109.024511 26.688501) (width 0.25) (layer "B.Cu") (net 8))
 (segment (start 109.903501 28.349511) (end 109.024511 27.470521) (width 0.25) (layer "B.Cu") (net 8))
 (segment (start 114.802216 30.889511) (end 112.443501 30.889511) (width 0.25) (layer "B.Cu") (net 8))
 (segment (start 112.443501 30.889511) (end 111.755489 30.201499) (width 0.25) (layer "B.Cu") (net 8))
 (segment (start 111.755489 29.228501) (end 110.876499 28.349511) (width 0.25) (layer "B.Cu") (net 8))
 (segment (start 110.876499 28.349511) (end 109.903501 28.349511) (width 0.25) (layer "B.Cu") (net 8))
 (segment (start 58.224031 31.339031) (end 56.6 29.715) (width 0.25) (layer "B.Cu") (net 8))
 (segment (start 66.755718 25.98) (end 61.396687 31.339031) (width 0.25) (layer "B.Cu") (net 8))
 (segment (start 111.755489 30.201499) (end 111.755489 29.228501) (width 0.25) (layer "B.Cu") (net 8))
 (segment (start 126.66098 30.99402) (end 127.94 29.715) (width 0.25) (layer "F.Cu") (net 9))
 (segment (start 124.98 32.28) (end 126.26598 30.99402) (width 0.25) (layer "F.Cu") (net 9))
 (segment (start 126.26598 30.99402) (end 126.66098 30.99402) (width 0.25) (layer "F.Cu") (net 9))
 (via (at 124.98 32.28) (size 0.8) (drill 0.4) (layers "F.Cu" "B.Cu") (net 9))
 (segment (start 110.353021 31.339031) (end 109.215489 30.201499) (width 0.25) (layer "B.Cu") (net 9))
 (segment (start 109.215489 29.228501) (end 108.336499 28.349511) (width 0.25) (layer "B.Cu") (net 9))
 (segment (start 109.215489 30.201499) (end 109.215489 29.228501) (width 0.25) (layer "B.Cu") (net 9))
 (segment (start 124.98 32.28) (end 124.488551 31.788551) (width 0.25) (layer "B.Cu") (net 9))
 (segment (start 56.133551 31.788551) (end 54.06 29.715) (width 0.25) (layer "B.Cu") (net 9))
 (segment (start 65.021924 28.349511) (end 61.582884 31.788551) (width 0.25) (layer "B.Cu") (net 9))
 (segment (start 108.336499 28.349511) (end 65.021924 28.349511) (width 0.25) (layer "B.Cu") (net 9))
 (segment (start 114.616018 31.339031) (end 110.353021 31.339031) (width 0.25) (layer "B.Cu") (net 9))
 (segment (start 61.582884 31.788551) (end 56.133551 31.788551) (width 0.25) (layer "B.Cu") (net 9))
 (segment (start 115.065538 31.788551) (end 114.616018 31.339031) (width 0.25) (layer "B.Cu") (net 9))
 (segment (start 124.488551 31.788551) (end 115.065538 31.788551) (width 0.25) (layer "B.Cu") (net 9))
 (segment (start 129.114511 29.228501) (end 128.426499 28.540489) (width 0.25) (layer "F.Cu") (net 10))
 (segment (start 128.426499 28.540489) (end 126.574511 28.540489) (width 0.25) (layer "F.Cu") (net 10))
 (segment (start 126.22 34.2) (end 129.114511 31.305489) (width 0.25) (layer "F.Cu") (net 10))
 (segment (start 129.114511 31.305489) (end 129.114511 29.228501) (width 0.25) (layer "F.Cu") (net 10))
 (segment (start 126.574511 28.540489) (end 125.4 29.715) (width 0.25) (layer "F.Cu") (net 10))
 (via (at 126.22 34.2) (size 0.8) (drill 0.4) (layers "F.Cu" "B.Cu") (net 10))
 (segment (start 47.11 33.24601) (end 50.64101 29.715) (width 0.25) (layer "B.Cu") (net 10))
 (segment (start 47.11 33.94) (end 47.11 33.24601) (width 0.25) (layer "B.Cu") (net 10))
 (segment (start 47.76 34.59) (end 47.11 33.94) (width 0.25) (layer "B.Cu") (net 10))
 (segment (start 50.64101 29.715) (end 51.52 29.715) (width 0.25) (layer "B.Cu") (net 10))
 (segment (start 126.22 34.2) (end 125.83 34.59) (width 0.25) (layer "B.Cu") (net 10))
 (segment (start 125.83 34.59) (end 47.76 34.59) (width 0.25) (layer "B.Cu") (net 10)))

